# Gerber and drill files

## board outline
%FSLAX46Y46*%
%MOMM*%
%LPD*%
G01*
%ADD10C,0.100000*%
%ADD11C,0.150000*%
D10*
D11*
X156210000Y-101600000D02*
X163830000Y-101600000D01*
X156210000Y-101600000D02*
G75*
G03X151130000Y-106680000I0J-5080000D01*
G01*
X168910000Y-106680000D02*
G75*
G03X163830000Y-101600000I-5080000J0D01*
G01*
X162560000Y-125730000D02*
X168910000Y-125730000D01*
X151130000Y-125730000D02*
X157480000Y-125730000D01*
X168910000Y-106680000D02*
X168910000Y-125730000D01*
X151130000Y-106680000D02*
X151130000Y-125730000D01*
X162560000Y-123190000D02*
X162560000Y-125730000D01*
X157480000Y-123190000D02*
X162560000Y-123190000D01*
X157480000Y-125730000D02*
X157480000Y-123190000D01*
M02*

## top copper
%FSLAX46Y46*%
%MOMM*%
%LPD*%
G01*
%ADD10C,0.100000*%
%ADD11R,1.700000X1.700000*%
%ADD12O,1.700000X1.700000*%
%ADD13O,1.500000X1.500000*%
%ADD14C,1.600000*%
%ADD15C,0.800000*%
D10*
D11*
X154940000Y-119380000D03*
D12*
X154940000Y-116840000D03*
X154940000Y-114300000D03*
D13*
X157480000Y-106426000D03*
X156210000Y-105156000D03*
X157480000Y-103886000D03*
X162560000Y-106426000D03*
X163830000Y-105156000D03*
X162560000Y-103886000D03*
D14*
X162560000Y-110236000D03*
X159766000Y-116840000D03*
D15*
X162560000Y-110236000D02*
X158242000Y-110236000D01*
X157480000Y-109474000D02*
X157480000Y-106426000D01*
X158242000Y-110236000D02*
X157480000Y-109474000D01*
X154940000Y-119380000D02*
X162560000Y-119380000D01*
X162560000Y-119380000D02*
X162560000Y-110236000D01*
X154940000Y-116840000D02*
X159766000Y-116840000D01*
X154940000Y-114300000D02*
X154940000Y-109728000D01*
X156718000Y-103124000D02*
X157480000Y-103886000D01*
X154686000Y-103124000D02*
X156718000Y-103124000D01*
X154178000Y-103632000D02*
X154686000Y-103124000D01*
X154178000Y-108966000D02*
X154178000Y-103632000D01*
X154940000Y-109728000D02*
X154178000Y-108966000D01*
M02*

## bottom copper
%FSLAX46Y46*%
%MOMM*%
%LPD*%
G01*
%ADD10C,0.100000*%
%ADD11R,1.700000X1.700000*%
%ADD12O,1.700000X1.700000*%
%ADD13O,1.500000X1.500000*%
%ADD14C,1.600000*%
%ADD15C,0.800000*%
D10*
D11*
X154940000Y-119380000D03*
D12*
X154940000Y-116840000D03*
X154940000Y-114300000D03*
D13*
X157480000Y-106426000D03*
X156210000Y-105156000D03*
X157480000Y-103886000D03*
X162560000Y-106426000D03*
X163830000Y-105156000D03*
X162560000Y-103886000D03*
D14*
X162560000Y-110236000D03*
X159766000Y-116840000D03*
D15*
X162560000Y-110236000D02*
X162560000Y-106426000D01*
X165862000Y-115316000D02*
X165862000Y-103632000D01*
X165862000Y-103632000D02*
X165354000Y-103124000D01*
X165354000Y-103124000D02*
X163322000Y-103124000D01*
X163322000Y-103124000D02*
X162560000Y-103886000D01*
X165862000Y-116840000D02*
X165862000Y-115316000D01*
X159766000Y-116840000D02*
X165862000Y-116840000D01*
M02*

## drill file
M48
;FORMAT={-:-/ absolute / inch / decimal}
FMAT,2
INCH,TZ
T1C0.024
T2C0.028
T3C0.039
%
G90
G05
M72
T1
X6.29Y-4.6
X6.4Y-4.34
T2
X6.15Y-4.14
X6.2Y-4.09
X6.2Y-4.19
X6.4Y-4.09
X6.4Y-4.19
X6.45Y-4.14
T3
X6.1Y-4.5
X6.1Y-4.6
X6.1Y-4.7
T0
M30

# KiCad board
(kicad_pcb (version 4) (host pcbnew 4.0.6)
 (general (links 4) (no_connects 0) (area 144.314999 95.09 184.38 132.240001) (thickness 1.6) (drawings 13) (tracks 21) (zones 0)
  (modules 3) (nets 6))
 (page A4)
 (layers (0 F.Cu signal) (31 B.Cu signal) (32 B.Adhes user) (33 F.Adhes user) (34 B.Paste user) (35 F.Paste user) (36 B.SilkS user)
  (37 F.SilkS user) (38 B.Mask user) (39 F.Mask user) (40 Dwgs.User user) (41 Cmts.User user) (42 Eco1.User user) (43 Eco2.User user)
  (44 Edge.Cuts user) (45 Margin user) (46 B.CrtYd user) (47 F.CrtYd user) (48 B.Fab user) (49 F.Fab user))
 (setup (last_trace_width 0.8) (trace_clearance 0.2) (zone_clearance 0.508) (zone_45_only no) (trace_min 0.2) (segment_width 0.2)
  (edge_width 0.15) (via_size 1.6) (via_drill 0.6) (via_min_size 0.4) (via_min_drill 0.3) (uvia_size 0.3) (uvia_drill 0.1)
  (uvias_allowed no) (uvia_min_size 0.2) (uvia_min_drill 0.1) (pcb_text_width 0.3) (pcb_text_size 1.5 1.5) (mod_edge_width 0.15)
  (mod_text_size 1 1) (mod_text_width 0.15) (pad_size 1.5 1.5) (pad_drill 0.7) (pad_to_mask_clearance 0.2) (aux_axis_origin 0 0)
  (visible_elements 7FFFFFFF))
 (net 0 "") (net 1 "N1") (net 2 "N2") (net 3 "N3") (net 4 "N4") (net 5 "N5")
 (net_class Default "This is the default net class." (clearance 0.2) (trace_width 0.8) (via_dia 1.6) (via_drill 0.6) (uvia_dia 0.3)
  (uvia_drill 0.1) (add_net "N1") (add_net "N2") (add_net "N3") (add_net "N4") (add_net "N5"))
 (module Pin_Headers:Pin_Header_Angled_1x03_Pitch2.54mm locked (layer F.Cu) (at 154.94 119.38 180)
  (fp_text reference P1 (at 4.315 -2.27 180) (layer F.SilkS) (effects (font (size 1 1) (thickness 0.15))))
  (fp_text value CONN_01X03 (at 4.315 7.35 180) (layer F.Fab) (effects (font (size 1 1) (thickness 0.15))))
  (pad 1 thru_hole rect (at 0 0 180) (size 1.7 1.7) (drill 1) (layers *.Cu *.Mask) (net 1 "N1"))
  (pad 2 thru_hole oval (at 0 2.54 180) (size 1.7 1.7) (drill 1) (layers *.Cu *.Mask) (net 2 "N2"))
  (pad 3 thru_hole oval (at 0 5.08 180) (size 1.7 1.7) (drill 1) (layers *.Cu *.Mask) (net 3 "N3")))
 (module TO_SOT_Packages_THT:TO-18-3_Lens (layer B.Cu) (at 157.48 106.426 90)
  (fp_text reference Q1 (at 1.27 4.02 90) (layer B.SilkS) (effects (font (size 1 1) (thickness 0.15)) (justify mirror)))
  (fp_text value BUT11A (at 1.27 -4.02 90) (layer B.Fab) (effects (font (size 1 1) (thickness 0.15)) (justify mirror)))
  (pad 3 thru_hole oval (at 0 0 90) (size 1.5 1.5) (drill 0.7) (layers *.Cu *.Mask) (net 1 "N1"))
  (pad 1 thru_hole oval (at 1.27 -1.27 90) (size 1.5 1.5) (drill 0.7) (layers *.Cu *.Mask) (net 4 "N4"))
  (pad 2 thru_hole oval (at 2.54 0 90) (size 1.5 1.5) (drill 0.7) (layers *.Cu *.Mask) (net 3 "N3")))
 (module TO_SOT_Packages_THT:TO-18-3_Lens (layer F.Cu) (at 162.56 106.426 90)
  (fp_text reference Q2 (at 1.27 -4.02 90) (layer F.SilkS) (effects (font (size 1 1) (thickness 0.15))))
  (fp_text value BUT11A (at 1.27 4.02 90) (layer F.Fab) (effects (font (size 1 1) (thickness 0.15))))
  (pad 3 thru_hole oval (at 0 0 90) (size 1.5 1.5) (drill 0.7) (layers *.Cu *.Mask) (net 1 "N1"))
  (pad 1 thru_hole oval (at 1.27 1.27 90) (size 1.5 1.5) (drill 0.7) (layers *.Cu *.Mask) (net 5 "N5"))
  (pad 2 thru_hole oval (at 2.54 0 90) (size 1.5 1.5) (drill 0.7) (layers *.Cu *.Mask) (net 2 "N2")))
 (gr_line (start 156.21 101.6) (end 163.83 101.6) (angle 90) (layer Edge.Cuts) (width 0.15))
 (gr_arc (start 156.21 106.68) (end 151.13 106.68) (angle 90) (layer Edge.Cuts) (width 0.15))
 (gr_arc (start 163.83 106.68) (end 163.83 101.6) (angle 90) (layer Edge.Cuts) (width 0.15))
 (gr_line (start 162.56 125.73) (end 168.91 125.73) (angle 90) (layer Edge.Cuts) (width 0.15))
 (gr_line (start 151.13 125.73) (end 157.48 125.73) (angle 90) (layer Edge.Cuts) (width 0.15))
 (gr_line (start 168.91 106.68) (end 168.91 125.73) (angle 90) (layer Edge.Cuts) (width 0.15))
 (gr_line (start 151.13 106.68) (end 151.13 125.73) (angle 90) (layer Edge.Cuts) (width 0.15))
 (gr_line (start 162.56 123.19) (end 162.56 125.73) (angle 90) (layer Edge.Cuts) (width 0.15))
 (gr_line (start 157.48 123.19) (end 162.56 123.19) (angle 90) (layer Edge.Cuts) (width 0.15))
 (gr_line (start 157.48 125.73) (end 157.48 123.19) (angle 90) (layer Edge.Cuts) (width 0.15))
 (segment (start 162.56 110.236) (end 158.242 110.236) (width 0.8) (layer F.Cu) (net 1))
 (segment (start 157.48 109.474) (end 157.48 106.426) (width 0.8) (layer F.Cu) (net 1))
 (segment (start 158.242 110.236) (end 157.48 109.474) (width 0.8) (layer F.Cu) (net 1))
 (segment (start 154.94 119.38) (end 162.56 119.38) (width 0.8) (layer F.Cu) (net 1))
 (segment (start 162.56 110.236) (end 162.56 106.426) (width 0.8) (layer B.Cu) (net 1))
 (via (at 162.56 110.236) (size 1.6) (drill 0.6) (layers F.Cu B.Cu) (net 1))
 (segment (start 162.56 119.38) (end 162.56 110.236) (width 0.8) (layer F.Cu) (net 1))
 (segment (start 154.94 116.84) (end 159.766 116.84) (width 0.8) (layer F.Cu) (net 2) (status 400000))
 (segment (start 165.862 115.316) (end 165.862 103.632) (width 0.8) (layer B.Cu) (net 2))
 (segment (start 165.862 103.632) (end 165.354 103.124) (width 0.8) (layer B.Cu) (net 2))
 (segment (start 165.354 103.124) (end 163.322 103.124) (width 0.8) (layer B.Cu) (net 2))
 (segment (start 163.322 103.124) (end 162.56 103.886) (width 0.8) (layer B.Cu) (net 2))
 (segment (start 165.862 116.84) (end 165.862 115.316) (width 0.8) (layer B.Cu) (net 2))
 (segment (start 159.766 116.84) (end 165.862 116.84) (width 0.8) (layer B.Cu) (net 2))
 (via (at 159.766 116.84) (size 1.6) (drill 0.6) (layers F.Cu B.Cu) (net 2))
 (segment (start 154.94 114.3) (end 154.94 109.728) (width 0.8) (layer F.Cu) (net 3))
 (segment (start 156.718 103.124) (end 157.48 103.886) (width 0.8) (layer F.Cu) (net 3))
 (segment (start 154.686 103.124) (end 156.718 103.124) (width 0.8) (layer F.Cu) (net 3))
 (segment (start 154.178 103.632) (end 154.686 103.124) (width 0.8) (layer F.Cu) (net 3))
 (segment (start 154.178 108.966) (end 154.178 103.632) (width 0.8) (layer F.Cu) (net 3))
 (segment (start 154.94 109.728) (end 154.178 108.966) (width 0.8) (layer F.Cu) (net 3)))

